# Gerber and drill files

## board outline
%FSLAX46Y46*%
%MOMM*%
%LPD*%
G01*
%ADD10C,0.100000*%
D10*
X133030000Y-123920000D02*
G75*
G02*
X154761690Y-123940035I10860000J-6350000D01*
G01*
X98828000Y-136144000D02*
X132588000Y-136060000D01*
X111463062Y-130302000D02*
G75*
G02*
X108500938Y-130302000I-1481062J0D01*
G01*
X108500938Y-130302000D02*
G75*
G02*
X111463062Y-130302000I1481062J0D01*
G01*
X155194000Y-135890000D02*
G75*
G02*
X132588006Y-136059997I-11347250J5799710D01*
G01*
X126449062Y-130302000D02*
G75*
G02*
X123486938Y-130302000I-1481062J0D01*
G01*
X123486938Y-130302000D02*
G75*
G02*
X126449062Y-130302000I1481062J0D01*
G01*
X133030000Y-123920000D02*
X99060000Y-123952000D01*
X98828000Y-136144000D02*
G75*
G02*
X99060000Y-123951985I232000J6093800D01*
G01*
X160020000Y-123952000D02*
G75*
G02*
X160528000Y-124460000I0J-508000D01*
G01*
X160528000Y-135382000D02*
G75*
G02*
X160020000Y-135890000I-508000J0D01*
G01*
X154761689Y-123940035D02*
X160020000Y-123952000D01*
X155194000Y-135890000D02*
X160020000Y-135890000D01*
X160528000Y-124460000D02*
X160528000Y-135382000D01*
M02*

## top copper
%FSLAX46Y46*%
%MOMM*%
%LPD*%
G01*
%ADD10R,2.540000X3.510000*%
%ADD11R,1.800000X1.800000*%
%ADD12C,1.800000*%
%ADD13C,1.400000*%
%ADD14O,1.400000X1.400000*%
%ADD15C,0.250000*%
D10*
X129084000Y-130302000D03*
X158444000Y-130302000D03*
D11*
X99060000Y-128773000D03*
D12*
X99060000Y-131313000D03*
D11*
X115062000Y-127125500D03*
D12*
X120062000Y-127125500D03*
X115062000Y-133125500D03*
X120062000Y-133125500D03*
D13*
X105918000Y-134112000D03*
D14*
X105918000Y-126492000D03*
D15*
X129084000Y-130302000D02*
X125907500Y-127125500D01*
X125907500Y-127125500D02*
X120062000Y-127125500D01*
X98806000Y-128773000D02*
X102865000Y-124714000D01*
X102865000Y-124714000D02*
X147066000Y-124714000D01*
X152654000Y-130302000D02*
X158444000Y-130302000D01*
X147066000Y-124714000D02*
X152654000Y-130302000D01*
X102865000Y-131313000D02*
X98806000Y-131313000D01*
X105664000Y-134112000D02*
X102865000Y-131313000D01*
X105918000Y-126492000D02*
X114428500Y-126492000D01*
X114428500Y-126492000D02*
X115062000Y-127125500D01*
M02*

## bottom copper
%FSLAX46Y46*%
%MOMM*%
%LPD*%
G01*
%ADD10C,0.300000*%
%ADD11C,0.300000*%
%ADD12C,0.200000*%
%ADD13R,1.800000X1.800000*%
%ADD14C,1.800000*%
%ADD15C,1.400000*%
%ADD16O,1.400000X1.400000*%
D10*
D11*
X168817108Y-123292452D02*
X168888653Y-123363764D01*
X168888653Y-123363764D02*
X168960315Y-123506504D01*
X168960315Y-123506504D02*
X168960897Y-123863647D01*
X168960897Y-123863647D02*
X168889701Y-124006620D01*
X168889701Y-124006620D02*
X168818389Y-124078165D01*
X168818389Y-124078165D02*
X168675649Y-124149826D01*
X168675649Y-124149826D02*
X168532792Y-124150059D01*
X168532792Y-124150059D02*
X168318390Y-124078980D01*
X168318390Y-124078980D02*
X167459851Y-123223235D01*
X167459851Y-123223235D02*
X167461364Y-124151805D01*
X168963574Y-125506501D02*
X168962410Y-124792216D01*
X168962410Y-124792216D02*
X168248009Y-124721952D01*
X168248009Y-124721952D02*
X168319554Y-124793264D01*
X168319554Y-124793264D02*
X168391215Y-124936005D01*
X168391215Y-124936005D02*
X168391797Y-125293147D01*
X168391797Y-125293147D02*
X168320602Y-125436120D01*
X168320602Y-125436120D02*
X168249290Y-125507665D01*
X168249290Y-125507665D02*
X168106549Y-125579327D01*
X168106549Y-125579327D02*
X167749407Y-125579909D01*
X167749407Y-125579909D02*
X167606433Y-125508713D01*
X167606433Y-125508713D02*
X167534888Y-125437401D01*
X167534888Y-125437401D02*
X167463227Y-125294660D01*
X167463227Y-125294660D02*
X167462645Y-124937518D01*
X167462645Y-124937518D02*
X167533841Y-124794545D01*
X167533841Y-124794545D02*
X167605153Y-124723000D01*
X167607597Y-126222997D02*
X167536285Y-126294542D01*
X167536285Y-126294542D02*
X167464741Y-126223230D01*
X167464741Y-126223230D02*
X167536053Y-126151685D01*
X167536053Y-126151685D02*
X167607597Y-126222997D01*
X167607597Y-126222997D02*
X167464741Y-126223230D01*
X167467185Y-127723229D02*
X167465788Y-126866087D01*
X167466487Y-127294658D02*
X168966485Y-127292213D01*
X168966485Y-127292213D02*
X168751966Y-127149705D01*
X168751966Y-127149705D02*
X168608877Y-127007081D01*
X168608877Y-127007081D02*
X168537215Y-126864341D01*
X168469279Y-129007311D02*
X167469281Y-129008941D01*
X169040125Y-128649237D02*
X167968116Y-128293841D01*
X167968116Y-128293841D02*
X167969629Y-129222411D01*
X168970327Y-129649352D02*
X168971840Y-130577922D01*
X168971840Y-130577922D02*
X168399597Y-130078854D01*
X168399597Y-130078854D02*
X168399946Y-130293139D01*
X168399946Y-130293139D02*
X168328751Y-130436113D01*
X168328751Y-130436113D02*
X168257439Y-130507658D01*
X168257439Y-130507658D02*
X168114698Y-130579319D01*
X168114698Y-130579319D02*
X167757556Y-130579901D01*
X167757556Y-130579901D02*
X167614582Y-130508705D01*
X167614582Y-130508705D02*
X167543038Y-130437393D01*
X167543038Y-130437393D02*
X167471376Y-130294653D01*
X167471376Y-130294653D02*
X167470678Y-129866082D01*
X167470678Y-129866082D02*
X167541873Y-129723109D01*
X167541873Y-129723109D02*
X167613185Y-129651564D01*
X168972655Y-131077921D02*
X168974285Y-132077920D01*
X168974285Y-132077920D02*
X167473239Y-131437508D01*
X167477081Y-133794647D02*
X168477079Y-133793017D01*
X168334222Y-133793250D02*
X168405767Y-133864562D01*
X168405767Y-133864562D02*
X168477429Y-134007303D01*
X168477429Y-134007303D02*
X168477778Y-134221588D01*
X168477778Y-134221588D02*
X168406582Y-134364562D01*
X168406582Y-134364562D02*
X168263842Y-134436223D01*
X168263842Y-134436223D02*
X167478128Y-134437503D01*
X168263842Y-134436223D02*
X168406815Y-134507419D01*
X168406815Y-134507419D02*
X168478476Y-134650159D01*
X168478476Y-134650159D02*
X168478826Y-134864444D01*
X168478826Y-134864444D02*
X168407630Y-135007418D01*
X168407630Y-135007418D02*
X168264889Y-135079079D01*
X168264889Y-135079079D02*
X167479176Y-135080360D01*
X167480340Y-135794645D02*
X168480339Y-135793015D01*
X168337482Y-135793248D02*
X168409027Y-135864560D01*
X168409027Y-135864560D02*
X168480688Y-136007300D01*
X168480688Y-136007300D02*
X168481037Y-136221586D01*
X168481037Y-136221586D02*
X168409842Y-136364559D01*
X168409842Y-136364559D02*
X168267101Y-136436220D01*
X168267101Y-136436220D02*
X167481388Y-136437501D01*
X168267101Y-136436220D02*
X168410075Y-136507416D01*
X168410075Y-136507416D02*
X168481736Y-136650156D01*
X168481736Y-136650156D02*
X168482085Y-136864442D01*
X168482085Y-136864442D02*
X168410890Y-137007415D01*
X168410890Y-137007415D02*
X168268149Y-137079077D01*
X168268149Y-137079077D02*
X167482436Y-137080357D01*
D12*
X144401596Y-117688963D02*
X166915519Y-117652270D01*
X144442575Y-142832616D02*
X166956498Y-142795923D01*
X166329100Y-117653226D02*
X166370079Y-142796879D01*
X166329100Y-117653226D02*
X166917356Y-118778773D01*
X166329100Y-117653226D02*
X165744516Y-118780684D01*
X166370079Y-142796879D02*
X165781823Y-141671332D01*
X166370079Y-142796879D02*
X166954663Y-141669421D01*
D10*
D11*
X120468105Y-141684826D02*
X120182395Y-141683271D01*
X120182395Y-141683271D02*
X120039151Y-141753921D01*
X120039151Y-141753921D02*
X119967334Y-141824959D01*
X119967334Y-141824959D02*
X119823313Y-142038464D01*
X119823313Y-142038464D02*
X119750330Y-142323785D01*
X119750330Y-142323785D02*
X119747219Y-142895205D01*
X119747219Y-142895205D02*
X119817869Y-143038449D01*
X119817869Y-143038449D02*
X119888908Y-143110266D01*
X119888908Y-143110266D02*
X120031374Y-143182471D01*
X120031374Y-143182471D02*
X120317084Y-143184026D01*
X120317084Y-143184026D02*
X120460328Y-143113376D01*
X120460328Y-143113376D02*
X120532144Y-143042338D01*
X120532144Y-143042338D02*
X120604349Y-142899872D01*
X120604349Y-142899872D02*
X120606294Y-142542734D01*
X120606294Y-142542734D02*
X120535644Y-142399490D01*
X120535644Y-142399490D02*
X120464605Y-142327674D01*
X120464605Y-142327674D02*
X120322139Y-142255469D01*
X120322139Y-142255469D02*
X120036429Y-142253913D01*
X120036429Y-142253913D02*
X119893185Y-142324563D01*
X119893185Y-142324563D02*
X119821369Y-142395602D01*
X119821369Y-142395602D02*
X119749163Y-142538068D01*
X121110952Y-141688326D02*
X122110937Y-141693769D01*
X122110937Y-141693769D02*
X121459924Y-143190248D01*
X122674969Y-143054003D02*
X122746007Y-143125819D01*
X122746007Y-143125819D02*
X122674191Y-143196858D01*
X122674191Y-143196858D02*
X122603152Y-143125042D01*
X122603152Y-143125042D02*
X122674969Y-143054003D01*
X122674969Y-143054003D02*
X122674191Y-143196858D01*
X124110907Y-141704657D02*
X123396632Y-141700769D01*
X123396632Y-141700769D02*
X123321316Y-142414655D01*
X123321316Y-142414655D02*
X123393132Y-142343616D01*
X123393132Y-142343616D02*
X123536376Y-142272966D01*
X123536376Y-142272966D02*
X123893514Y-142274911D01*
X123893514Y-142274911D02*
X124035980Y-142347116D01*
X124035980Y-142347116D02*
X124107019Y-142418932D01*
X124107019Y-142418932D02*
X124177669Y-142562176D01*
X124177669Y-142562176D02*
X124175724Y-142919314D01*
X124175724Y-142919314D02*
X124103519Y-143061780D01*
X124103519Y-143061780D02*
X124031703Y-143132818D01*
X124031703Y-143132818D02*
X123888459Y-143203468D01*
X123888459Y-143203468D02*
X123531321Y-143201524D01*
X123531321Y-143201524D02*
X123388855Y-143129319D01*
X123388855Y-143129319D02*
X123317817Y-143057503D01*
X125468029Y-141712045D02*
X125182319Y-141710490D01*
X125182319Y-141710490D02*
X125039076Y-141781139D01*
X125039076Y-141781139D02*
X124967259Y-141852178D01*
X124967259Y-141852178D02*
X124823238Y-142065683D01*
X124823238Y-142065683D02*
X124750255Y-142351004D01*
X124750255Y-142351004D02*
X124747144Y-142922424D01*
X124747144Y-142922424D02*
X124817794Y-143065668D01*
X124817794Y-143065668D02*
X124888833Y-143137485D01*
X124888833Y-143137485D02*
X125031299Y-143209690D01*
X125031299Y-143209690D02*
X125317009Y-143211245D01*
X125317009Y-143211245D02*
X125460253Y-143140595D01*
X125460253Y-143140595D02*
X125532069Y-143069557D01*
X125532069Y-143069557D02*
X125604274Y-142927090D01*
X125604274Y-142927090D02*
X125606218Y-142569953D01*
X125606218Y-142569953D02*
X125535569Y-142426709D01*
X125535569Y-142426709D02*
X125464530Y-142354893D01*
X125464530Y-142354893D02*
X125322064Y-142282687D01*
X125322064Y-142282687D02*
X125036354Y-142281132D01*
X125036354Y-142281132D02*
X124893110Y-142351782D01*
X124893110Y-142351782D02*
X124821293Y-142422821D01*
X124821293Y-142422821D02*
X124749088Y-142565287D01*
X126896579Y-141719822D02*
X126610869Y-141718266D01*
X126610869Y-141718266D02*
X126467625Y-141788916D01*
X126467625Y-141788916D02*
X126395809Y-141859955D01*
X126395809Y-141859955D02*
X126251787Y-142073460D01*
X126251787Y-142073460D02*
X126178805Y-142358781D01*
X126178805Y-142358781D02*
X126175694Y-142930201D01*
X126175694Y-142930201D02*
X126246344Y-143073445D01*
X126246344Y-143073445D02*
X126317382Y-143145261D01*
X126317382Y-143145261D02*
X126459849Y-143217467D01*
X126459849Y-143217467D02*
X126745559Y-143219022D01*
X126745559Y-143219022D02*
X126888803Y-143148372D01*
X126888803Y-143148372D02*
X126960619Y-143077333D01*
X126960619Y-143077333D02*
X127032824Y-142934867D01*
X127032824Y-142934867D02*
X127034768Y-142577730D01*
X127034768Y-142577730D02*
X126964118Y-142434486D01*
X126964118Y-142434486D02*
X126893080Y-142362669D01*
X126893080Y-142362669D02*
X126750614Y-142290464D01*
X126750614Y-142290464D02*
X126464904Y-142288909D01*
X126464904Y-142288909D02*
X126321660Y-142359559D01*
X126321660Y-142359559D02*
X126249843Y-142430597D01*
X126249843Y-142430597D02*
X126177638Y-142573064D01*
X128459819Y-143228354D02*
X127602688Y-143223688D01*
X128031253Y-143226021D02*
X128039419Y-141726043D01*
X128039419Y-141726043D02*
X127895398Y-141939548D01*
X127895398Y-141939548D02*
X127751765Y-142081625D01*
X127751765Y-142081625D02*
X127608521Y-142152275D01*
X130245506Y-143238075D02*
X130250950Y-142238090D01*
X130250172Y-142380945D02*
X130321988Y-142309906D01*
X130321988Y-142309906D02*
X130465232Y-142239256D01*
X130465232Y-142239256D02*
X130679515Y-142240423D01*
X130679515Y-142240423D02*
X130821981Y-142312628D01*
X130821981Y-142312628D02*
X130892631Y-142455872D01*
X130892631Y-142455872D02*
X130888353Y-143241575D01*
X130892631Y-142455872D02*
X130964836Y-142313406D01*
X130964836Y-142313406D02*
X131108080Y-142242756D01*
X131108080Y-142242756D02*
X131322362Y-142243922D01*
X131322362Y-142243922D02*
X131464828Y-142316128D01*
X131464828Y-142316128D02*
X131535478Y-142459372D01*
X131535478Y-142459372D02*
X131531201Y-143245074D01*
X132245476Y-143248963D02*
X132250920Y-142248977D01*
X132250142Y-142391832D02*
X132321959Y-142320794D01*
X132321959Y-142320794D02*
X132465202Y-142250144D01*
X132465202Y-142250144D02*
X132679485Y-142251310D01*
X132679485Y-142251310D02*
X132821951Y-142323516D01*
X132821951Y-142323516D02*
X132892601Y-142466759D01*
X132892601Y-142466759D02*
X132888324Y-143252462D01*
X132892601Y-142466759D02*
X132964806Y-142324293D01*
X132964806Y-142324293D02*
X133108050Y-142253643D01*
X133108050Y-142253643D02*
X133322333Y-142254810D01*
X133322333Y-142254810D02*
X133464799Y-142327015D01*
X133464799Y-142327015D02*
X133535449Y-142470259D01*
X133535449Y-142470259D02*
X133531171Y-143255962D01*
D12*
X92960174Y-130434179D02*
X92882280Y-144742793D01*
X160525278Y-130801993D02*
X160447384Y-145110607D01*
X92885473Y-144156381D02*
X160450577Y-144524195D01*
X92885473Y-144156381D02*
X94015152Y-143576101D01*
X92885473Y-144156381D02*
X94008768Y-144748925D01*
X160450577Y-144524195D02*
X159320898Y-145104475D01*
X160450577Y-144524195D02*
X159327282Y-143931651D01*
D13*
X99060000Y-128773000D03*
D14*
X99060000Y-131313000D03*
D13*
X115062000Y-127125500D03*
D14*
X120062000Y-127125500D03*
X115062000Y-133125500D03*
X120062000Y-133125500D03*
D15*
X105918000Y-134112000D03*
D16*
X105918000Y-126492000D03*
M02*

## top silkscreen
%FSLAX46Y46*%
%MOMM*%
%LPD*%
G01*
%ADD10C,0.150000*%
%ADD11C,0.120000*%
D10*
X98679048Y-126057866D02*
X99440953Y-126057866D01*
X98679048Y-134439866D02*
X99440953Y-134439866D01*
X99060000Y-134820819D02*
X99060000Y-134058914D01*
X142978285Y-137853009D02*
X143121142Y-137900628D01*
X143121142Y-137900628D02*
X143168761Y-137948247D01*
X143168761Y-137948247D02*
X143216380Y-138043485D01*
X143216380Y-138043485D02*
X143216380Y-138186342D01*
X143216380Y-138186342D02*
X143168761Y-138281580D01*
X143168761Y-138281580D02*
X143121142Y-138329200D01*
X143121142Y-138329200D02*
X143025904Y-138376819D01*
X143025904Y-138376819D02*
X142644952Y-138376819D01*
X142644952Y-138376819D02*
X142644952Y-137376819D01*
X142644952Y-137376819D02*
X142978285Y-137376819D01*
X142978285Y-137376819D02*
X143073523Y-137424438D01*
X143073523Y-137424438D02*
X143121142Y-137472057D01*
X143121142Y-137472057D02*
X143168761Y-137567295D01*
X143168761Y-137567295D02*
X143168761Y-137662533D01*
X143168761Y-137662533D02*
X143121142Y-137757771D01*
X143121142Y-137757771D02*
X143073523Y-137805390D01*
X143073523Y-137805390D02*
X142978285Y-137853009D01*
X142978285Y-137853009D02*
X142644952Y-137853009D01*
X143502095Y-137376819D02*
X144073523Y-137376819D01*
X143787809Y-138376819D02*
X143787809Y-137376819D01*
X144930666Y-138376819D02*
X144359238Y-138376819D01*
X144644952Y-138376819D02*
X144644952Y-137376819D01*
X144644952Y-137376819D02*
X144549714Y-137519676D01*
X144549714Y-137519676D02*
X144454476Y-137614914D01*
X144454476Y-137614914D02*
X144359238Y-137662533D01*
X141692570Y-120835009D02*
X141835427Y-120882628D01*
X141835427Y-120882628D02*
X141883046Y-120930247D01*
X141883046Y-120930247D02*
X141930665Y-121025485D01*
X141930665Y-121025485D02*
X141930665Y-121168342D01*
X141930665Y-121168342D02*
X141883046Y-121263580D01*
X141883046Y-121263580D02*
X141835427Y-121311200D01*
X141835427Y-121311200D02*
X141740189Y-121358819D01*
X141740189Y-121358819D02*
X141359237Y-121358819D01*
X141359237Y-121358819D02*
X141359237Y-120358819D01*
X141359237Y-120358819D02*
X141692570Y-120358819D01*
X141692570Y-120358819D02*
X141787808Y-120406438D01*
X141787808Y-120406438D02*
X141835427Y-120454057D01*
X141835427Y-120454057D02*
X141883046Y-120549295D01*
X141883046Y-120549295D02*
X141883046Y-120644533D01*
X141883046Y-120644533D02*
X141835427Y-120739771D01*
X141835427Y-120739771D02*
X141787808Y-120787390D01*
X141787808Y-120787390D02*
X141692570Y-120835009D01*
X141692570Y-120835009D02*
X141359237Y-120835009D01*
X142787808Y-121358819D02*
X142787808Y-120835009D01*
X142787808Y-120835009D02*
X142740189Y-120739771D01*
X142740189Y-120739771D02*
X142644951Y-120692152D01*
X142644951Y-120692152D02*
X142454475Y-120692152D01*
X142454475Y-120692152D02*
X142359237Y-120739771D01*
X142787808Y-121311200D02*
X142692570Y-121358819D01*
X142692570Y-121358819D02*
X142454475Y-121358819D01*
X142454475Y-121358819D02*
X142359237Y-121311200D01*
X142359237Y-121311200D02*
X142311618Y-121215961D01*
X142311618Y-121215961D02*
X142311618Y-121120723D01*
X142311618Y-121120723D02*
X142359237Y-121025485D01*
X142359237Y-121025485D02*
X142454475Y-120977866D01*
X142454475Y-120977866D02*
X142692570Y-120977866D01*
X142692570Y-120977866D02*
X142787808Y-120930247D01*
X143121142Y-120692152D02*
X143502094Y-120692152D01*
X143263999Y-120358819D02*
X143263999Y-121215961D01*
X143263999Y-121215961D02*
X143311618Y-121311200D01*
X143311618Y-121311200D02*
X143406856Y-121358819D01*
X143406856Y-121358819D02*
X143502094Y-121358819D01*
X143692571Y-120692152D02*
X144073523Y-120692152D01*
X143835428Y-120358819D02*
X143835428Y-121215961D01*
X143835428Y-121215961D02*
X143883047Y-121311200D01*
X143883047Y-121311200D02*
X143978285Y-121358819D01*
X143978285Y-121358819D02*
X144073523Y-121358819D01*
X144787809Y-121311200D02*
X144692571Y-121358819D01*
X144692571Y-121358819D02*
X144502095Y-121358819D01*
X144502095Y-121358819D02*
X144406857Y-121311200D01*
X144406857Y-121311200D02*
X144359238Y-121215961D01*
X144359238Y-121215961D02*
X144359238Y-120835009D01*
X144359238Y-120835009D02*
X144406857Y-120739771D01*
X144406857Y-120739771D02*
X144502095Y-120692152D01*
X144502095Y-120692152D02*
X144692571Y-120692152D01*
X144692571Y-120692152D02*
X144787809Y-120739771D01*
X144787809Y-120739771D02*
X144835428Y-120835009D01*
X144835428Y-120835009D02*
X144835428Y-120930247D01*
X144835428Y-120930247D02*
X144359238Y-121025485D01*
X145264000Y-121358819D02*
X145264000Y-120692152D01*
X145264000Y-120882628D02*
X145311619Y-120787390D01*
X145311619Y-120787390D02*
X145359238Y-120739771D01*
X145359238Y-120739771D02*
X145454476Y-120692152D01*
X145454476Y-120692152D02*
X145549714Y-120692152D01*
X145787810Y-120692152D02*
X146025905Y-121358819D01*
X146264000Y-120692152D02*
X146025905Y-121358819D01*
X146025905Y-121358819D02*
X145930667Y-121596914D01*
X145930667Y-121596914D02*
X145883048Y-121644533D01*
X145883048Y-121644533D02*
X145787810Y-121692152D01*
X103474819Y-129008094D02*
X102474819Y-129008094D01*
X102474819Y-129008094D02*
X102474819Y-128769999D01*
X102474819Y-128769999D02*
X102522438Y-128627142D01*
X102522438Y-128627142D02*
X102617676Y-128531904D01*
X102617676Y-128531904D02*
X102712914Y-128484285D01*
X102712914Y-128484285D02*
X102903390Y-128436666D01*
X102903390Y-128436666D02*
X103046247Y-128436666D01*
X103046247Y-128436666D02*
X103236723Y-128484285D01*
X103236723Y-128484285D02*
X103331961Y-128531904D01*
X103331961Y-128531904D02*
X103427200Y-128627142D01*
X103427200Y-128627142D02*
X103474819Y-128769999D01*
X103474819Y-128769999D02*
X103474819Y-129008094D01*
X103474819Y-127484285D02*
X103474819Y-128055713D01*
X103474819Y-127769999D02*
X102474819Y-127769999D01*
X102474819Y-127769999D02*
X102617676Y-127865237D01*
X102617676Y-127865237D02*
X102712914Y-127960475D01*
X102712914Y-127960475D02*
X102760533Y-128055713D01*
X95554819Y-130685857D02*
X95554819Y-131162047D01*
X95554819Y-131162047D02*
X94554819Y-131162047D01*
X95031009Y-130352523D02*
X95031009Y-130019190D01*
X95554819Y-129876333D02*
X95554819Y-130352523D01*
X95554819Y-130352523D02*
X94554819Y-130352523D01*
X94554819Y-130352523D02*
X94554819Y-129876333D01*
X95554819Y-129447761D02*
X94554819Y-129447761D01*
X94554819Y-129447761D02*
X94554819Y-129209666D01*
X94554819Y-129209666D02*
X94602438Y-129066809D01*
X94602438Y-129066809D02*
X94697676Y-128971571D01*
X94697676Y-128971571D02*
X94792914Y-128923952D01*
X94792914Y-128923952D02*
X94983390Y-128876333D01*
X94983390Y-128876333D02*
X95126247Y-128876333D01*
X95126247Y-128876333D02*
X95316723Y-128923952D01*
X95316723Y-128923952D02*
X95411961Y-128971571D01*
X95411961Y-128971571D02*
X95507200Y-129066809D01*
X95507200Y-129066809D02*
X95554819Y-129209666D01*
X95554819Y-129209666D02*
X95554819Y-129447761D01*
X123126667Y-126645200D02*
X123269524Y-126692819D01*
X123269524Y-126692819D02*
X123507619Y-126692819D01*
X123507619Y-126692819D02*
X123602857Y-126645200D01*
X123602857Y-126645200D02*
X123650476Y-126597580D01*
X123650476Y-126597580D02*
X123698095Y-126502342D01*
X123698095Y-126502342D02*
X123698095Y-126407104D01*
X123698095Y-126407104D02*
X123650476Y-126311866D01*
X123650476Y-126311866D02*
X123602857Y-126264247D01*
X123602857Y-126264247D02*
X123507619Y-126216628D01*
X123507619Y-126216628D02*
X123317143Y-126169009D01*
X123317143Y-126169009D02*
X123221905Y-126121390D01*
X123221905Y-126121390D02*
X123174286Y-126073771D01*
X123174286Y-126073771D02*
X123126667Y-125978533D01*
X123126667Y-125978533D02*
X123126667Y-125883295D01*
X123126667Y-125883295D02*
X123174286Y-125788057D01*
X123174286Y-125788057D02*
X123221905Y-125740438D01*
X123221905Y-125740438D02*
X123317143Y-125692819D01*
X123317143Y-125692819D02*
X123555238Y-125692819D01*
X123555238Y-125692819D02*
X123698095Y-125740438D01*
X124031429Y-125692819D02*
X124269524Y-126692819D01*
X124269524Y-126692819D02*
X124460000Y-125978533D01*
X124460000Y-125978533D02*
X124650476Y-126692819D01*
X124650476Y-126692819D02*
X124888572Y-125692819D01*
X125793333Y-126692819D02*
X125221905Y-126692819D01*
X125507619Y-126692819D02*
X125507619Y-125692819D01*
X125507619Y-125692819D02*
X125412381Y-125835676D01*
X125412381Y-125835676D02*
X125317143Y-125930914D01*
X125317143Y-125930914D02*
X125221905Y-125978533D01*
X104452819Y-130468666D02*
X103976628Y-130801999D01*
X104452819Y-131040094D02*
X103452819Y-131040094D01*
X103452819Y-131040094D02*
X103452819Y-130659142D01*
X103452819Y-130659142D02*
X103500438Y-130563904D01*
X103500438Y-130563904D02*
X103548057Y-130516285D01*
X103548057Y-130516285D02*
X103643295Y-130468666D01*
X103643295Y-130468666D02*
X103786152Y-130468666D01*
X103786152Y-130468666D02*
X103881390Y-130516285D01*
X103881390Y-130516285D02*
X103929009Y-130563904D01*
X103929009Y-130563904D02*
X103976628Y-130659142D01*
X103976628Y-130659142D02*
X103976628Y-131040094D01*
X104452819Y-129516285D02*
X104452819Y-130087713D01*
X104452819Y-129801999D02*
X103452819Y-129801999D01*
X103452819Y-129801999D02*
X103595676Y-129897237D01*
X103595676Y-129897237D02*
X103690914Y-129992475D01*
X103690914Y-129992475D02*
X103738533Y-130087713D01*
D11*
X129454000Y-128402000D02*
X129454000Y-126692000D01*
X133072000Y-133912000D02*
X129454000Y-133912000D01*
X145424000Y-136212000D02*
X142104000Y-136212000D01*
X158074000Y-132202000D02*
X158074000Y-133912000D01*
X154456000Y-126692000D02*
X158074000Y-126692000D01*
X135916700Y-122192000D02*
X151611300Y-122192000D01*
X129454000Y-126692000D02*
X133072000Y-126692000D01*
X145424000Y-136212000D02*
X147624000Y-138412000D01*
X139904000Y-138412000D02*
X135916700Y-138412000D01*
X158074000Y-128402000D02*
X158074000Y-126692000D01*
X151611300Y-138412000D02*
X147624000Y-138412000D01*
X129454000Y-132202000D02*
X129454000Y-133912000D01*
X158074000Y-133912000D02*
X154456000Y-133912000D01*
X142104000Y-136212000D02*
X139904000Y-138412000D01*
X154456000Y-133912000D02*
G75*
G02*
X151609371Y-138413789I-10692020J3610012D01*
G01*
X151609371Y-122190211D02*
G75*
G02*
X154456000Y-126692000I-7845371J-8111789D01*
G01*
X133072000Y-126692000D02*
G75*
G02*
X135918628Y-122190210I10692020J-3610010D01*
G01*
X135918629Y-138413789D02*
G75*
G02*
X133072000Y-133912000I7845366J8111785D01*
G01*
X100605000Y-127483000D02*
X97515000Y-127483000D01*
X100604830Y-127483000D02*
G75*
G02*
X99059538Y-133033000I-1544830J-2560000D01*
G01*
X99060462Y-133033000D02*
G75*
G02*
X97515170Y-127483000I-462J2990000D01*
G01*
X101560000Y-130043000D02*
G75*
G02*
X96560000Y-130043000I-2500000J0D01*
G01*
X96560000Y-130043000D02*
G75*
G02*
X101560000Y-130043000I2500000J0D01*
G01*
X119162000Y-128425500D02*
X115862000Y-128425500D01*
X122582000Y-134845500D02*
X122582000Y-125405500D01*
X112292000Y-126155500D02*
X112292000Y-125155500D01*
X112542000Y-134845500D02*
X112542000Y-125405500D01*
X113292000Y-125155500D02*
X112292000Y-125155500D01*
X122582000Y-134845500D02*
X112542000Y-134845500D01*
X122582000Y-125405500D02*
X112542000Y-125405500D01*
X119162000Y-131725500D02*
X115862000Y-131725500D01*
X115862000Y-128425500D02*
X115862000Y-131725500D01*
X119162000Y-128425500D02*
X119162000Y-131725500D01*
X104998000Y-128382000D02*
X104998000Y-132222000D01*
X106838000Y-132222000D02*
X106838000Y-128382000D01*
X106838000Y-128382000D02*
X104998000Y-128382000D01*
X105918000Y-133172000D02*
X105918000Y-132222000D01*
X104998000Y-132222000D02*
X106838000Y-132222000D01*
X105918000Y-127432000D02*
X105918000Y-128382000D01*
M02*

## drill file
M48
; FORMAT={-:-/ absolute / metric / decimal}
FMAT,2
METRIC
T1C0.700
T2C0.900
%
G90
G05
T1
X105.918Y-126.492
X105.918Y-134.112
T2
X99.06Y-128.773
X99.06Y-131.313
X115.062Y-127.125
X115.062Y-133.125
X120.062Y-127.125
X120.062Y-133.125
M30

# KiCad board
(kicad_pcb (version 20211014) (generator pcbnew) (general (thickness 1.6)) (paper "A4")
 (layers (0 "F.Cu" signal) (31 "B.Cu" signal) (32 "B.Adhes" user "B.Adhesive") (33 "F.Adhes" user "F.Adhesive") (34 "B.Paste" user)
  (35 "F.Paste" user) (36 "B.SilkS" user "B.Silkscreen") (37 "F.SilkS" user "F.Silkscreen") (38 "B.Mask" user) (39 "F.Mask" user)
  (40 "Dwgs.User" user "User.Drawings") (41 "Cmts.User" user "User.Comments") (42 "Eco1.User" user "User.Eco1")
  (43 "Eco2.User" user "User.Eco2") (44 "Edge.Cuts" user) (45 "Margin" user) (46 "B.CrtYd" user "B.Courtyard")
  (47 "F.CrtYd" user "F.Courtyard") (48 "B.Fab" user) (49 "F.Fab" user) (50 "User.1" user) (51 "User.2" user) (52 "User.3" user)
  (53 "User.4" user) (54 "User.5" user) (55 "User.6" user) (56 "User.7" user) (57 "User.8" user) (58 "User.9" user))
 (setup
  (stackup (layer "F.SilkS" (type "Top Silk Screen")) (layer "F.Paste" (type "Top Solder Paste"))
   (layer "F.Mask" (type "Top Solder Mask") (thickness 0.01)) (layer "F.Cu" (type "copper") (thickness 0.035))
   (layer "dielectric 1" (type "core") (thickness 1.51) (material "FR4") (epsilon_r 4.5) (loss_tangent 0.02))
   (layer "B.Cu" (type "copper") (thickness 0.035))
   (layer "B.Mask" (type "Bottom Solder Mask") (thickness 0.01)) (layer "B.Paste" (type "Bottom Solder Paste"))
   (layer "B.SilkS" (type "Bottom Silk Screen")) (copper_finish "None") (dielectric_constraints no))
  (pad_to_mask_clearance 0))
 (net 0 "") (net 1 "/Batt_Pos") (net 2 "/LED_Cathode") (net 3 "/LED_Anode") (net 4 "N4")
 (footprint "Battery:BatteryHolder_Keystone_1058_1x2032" (layer "F.Cu") (at 143.764 130.302)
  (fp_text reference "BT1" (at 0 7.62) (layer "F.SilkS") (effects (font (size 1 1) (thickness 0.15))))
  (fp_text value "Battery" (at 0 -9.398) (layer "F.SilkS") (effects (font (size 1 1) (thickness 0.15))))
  (fp_line (start -14.31 -1.9) (end -14.31 -3.61) (layer "F.SilkS") (width 0.12))
  (fp_line (start -10.692 3.61) (end -14.31 3.61) (layer "F.SilkS") (width 0.12))
  (fp_line (start 1.66 5.91) (end -1.66 5.91) (layer "F.SilkS") (width 0.12))
  (fp_line (start 14.31 1.9) (end 14.31 3.61) (layer "F.SilkS") (width 0.12))
  (fp_line (start 10.692 -3.61) (end 14.31 -3.61) (layer "F.SilkS") (width 0.12))
  (fp_line (start -7.8473 -8.11) (end 7.8473 -8.11) (layer "F.SilkS") (width 0.12))
  (fp_line (start -14.31 -3.61) (end -10.692 -3.61) (layer "F.SilkS") (width 0.12))
  (fp_line (start 1.66 5.91) (end 3.86 8.11) (layer "F.SilkS") (width 0.12))
  (fp_line (start -3.86 8.11) (end -7.8473 8.11) (layer "F.SilkS") (width 0.12))
  (fp_line (start 14.31 -1.9) (end 14.31 -3.61) (layer "F.SilkS") (width 0.12))
  (fp_line (start 7.8473 8.11) (end 3.86 8.11) (layer "F.SilkS") (width 0.12))
  (fp_line (start -14.31 1.9) (end -14.31 3.61) (layer "F.SilkS") (width 0.12))
  (fp_line (start 14.31 3.61) (end 10.692 3.61) (layer "F.SilkS") (width 0.12))
  (fp_line (start -1.66 5.91) (end -3.86 8.11) (layer "F.SilkS") (width 0.12))
  (fp_arc (start 10.692 3.61) (mid 9.538084 6.031244) (end 7.845371 8.111789) (layer "F.SilkS") (width 0.12))
  (fp_arc (start 7.845371 -8.111789) (mid 9.538085 -6.031244) (end 10.692 -3.61) (layer "F.SilkS") (width 0.12))
  (fp_arc (start -10.692 -3.61) (mid -9.538084 -6.031244) (end -7.845371 -8.111789) (layer "F.SilkS") (width 0.12))
  (fp_arc (start -7.845371 8.111789) (mid -9.538085 6.031244) (end -10.692 3.61) (layer "F.SilkS") (width 0.12))
  (pad "1" smd rect (at -14.68 0) (size 2.54 3.51) (layers "F.Cu" "F.Paste" "F.Mask") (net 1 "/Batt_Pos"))
  (pad "2" smd rect (at 14.68 0) (size 2.54 3.51) (layers "F.Cu" "F.Paste" "F.Mask") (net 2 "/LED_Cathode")))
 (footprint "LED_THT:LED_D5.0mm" (layer "F.Cu") (at 99.06 128.773 -90)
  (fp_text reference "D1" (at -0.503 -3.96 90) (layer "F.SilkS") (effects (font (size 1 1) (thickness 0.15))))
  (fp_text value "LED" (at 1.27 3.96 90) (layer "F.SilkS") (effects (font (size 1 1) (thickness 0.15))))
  (fp_line (start -1.29 -1.545) (end -1.29 1.545) (layer "F.SilkS") (width 0.12))
  (fp_arc (start -1.29 -1.54483) (mid 2.072002 -2.880433) (end 4.26 0.000462) (layer "F.SilkS") (width 0.12))
  (fp_arc (start 4.26 -0.000462) (mid 2.072002 2.880433) (end -1.29 1.54483) (layer "F.SilkS") (width 0.12))
  (fp_circle (center 1.27 0) (end 3.77 0) (layer "F.SilkS") (width 0.12) (fill none))
  (pad "1" thru_hole rect (at 0 0 270) (size 1.8 1.8) (drill 0.9) (layers *.Cu *.Mask) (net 2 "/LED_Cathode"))
  (pad "2" thru_hole circle (at 2.54 0 270) (size 1.8 1.8) (drill 0.9) (layers *.Cu *.Mask) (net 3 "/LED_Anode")))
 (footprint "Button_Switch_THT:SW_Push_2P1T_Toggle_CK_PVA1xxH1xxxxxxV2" (layer "F.Cu") (at 115.062 127.1255)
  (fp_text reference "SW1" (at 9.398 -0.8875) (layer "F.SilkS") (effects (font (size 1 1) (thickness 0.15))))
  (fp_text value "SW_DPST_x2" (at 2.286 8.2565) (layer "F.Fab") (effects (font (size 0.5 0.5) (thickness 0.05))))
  (fp_line (start 4.1 1.3) (end 0.8 1.3) (layer "F.SilkS") (width 0.12))
  (fp_line (start 7.52 7.72) (end 7.52 -1.72) (layer "F.SilkS") (width 0.12))
  (fp_line (start -2.77 -0.97) (end -2.77 -1.97) (layer "F.SilkS") (width 0.12))
  (fp_line (start -2.52 7.72) (end -2.52 -1.72) (layer "F.SilkS") (width 0.12))
  (fp_line (start -1.77 -1.97) (end -2.77 -1.97) (layer "F.SilkS") (width 0.12))
  (fp_line (start 7.52 7.72) (end -2.52 7.72) (layer "F.SilkS") (width 0.12))
  (fp_line (start 7.52 -1.72) (end -2.52 -1.72) (layer "F.SilkS") (width 0.12))
  (fp_line (start 4.1 4.6) (end 0.8 4.6) (layer "F.SilkS") (width 0.12))
  (fp_line (start 0.8 1.3) (end 0.8 4.6) (layer "F.SilkS") (width 0.12))
  (fp_line (start 4.1 1.3) (end 4.1 4.6) (layer "F.SilkS") (width 0.12))
  (pad "1" thru_hole rect (at 0 0) (size 1.8 1.8) (drill 0.9) (layers *.Cu *.Mask) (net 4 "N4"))
  (pad "2" thru_hole circle (at 5 0) (size 1.8 1.8) (drill 0.9) (layers *.Cu *.Mask) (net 1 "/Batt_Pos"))
  (pad "3" thru_hole circle (at 0 6) (size 1.8 1.8) (drill 0.9) (layers *.Cu *.Mask))
  (pad "4" thru_hole circle (at 5 6) (size 1.8 1.8) (drill 0.9) (layers *.Cu *.Mask)))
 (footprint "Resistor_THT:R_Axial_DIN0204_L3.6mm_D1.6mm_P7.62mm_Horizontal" (layer "F.Cu") (at 105.918 134.112 90)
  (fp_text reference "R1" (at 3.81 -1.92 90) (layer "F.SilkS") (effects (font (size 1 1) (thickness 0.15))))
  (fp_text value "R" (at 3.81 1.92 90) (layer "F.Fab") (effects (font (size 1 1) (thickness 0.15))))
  (fp_line (start 5.73 -0.92) (end 1.89 -0.92) (layer "F.SilkS") (width 0.12))
  (fp_line (start 1.89 0.92) (end 5.73 0.92) (layer "F.SilkS") (width 0.12))
  (fp_line (start 5.73 0.92) (end 5.73 -0.92) (layer "F.SilkS") (width 0.12))
  (fp_line (start 0.94 0) (end 1.89 0) (layer "F.SilkS") (width 0.12))
  (fp_line (start 1.89 -0.92) (end 1.89 0.92) (layer "F.SilkS") (width 0.12))
  (fp_line (start 6.68 0) (end 5.73 0) (layer "F.SilkS") (width 0.12))
  (pad "1" thru_hole circle (at 0 0 90) (size 1.4 1.4) (drill 0.7) (layers *.Cu *.Mask) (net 3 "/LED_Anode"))
  (pad "2" thru_hole oval (at 7.62 0 90) (size 1.4 1.4) (drill 0.7) (layers *.Cu *.Mask) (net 4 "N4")))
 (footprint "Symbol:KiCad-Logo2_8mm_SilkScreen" (layer "B.Cu") (at 143.764 130.302 180)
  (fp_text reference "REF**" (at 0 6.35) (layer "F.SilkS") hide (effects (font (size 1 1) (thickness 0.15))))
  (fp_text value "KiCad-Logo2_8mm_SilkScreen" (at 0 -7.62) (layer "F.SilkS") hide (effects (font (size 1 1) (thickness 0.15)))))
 (gr_arc (start 133.03 123.92) (mid 143.901597 117.689778) (end 154.761689 123.940035) (layer "Edge.Cuts") (width 0.1))
 (gr_line (start 98.828 136.144) (end 132.588 136.06) (layer "Edge.Cuts") (width 0.1))
 (gr_circle (center 109.982 130.302) (end 110.744 129.032) (layer "Edge.Cuts") (width 0.1) (fill none))
 (gr_arc (start 155.194 135.89) (mid 143.942576 142.833431) (end 132.588 136.06) (layer "Edge.Cuts") (width 0.1))
 (gr_circle (center 124.968 130.302) (end 125.73 129.032) (layer "Edge.Cuts") (width 0.1) (fill none))
 (gr_line (start 133.03 123.92) (end 99.06 123.952) (layer "Edge.Cuts") (width 0.1))
 (gr_arc (start 98.828 136.144) (mid 92.962896 129.934186) (end 99.06 123.952) (layer "Edge.Cuts") (width 0.1))
 (gr_arc (start 160.02 123.952) (mid 160.37921 124.10079) (end 160.528 124.46) (layer "Edge.Cuts") (width 0.1))
 (gr_arc (start 160.528 135.382) (mid 160.37921 135.74121) (end 160.02 135.89) (layer "Edge.Cuts") (width 0.1))
 (gr_line (start 154.761689 123.940035) (end 160.02 123.952) (layer "Edge.Cuts") (width 0.1))
 (gr_line (start 155.194 135.89) (end 160.02 135.89) (layer "Edge.Cuts") (width 0.1))
 (gr_line (start 160.528 124.46) (end 160.528 135.382) (layer "Edge.Cuts") (width 0.1))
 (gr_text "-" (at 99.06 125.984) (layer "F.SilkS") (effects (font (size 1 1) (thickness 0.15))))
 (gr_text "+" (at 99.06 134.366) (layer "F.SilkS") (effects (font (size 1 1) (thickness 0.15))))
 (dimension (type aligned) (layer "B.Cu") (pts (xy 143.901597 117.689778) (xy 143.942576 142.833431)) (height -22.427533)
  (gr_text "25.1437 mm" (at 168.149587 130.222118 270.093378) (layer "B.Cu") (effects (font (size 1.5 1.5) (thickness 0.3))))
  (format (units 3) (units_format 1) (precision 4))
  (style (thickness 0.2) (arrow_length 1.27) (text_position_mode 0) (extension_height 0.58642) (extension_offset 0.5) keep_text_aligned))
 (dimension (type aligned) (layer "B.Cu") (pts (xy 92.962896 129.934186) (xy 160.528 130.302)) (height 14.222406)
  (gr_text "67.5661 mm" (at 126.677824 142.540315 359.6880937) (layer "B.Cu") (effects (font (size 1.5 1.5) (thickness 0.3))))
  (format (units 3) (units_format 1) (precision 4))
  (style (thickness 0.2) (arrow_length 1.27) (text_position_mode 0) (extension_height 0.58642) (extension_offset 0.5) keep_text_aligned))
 (segment (start 129.084 130.302) (end 125.9075 127.1255) (width 0.25) (layer "F.Cu") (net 1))
 (segment (start 125.9075 127.1255) (end 120.062 127.1255) (width 0.25) (layer "F.Cu") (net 1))
 (segment (start 98.806 128.773) (end 102.865 124.714) (width 0.25) (layer "F.Cu") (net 2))
 (segment (start 102.865 124.714) (end 147.066 124.714) (width 0.25) (layer "F.Cu") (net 2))
 (segment (start 152.654 130.302) (end 158.444 130.302) (width 0.25) (layer "F.Cu") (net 2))
 (segment (start 147.066 124.714) (end 152.654 130.302) (width 0.25) (layer "F.Cu") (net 2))
 (segment (start 102.865 131.313) (end 98.806 131.313) (width 0.25) (layer "F.Cu") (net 3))
 (segment (start 105.664 134.112) (end 102.865 131.313) (width 0.25) (layer "F.Cu") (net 3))
 (segment (start 105.918 126.492) (end 114.4285 126.492) (width 0.25) (layer "F.Cu") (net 4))
 (segment (start 114.4285 126.492) (end 115.062 127.1255) (width 0.25) (layer "F.Cu") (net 4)))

